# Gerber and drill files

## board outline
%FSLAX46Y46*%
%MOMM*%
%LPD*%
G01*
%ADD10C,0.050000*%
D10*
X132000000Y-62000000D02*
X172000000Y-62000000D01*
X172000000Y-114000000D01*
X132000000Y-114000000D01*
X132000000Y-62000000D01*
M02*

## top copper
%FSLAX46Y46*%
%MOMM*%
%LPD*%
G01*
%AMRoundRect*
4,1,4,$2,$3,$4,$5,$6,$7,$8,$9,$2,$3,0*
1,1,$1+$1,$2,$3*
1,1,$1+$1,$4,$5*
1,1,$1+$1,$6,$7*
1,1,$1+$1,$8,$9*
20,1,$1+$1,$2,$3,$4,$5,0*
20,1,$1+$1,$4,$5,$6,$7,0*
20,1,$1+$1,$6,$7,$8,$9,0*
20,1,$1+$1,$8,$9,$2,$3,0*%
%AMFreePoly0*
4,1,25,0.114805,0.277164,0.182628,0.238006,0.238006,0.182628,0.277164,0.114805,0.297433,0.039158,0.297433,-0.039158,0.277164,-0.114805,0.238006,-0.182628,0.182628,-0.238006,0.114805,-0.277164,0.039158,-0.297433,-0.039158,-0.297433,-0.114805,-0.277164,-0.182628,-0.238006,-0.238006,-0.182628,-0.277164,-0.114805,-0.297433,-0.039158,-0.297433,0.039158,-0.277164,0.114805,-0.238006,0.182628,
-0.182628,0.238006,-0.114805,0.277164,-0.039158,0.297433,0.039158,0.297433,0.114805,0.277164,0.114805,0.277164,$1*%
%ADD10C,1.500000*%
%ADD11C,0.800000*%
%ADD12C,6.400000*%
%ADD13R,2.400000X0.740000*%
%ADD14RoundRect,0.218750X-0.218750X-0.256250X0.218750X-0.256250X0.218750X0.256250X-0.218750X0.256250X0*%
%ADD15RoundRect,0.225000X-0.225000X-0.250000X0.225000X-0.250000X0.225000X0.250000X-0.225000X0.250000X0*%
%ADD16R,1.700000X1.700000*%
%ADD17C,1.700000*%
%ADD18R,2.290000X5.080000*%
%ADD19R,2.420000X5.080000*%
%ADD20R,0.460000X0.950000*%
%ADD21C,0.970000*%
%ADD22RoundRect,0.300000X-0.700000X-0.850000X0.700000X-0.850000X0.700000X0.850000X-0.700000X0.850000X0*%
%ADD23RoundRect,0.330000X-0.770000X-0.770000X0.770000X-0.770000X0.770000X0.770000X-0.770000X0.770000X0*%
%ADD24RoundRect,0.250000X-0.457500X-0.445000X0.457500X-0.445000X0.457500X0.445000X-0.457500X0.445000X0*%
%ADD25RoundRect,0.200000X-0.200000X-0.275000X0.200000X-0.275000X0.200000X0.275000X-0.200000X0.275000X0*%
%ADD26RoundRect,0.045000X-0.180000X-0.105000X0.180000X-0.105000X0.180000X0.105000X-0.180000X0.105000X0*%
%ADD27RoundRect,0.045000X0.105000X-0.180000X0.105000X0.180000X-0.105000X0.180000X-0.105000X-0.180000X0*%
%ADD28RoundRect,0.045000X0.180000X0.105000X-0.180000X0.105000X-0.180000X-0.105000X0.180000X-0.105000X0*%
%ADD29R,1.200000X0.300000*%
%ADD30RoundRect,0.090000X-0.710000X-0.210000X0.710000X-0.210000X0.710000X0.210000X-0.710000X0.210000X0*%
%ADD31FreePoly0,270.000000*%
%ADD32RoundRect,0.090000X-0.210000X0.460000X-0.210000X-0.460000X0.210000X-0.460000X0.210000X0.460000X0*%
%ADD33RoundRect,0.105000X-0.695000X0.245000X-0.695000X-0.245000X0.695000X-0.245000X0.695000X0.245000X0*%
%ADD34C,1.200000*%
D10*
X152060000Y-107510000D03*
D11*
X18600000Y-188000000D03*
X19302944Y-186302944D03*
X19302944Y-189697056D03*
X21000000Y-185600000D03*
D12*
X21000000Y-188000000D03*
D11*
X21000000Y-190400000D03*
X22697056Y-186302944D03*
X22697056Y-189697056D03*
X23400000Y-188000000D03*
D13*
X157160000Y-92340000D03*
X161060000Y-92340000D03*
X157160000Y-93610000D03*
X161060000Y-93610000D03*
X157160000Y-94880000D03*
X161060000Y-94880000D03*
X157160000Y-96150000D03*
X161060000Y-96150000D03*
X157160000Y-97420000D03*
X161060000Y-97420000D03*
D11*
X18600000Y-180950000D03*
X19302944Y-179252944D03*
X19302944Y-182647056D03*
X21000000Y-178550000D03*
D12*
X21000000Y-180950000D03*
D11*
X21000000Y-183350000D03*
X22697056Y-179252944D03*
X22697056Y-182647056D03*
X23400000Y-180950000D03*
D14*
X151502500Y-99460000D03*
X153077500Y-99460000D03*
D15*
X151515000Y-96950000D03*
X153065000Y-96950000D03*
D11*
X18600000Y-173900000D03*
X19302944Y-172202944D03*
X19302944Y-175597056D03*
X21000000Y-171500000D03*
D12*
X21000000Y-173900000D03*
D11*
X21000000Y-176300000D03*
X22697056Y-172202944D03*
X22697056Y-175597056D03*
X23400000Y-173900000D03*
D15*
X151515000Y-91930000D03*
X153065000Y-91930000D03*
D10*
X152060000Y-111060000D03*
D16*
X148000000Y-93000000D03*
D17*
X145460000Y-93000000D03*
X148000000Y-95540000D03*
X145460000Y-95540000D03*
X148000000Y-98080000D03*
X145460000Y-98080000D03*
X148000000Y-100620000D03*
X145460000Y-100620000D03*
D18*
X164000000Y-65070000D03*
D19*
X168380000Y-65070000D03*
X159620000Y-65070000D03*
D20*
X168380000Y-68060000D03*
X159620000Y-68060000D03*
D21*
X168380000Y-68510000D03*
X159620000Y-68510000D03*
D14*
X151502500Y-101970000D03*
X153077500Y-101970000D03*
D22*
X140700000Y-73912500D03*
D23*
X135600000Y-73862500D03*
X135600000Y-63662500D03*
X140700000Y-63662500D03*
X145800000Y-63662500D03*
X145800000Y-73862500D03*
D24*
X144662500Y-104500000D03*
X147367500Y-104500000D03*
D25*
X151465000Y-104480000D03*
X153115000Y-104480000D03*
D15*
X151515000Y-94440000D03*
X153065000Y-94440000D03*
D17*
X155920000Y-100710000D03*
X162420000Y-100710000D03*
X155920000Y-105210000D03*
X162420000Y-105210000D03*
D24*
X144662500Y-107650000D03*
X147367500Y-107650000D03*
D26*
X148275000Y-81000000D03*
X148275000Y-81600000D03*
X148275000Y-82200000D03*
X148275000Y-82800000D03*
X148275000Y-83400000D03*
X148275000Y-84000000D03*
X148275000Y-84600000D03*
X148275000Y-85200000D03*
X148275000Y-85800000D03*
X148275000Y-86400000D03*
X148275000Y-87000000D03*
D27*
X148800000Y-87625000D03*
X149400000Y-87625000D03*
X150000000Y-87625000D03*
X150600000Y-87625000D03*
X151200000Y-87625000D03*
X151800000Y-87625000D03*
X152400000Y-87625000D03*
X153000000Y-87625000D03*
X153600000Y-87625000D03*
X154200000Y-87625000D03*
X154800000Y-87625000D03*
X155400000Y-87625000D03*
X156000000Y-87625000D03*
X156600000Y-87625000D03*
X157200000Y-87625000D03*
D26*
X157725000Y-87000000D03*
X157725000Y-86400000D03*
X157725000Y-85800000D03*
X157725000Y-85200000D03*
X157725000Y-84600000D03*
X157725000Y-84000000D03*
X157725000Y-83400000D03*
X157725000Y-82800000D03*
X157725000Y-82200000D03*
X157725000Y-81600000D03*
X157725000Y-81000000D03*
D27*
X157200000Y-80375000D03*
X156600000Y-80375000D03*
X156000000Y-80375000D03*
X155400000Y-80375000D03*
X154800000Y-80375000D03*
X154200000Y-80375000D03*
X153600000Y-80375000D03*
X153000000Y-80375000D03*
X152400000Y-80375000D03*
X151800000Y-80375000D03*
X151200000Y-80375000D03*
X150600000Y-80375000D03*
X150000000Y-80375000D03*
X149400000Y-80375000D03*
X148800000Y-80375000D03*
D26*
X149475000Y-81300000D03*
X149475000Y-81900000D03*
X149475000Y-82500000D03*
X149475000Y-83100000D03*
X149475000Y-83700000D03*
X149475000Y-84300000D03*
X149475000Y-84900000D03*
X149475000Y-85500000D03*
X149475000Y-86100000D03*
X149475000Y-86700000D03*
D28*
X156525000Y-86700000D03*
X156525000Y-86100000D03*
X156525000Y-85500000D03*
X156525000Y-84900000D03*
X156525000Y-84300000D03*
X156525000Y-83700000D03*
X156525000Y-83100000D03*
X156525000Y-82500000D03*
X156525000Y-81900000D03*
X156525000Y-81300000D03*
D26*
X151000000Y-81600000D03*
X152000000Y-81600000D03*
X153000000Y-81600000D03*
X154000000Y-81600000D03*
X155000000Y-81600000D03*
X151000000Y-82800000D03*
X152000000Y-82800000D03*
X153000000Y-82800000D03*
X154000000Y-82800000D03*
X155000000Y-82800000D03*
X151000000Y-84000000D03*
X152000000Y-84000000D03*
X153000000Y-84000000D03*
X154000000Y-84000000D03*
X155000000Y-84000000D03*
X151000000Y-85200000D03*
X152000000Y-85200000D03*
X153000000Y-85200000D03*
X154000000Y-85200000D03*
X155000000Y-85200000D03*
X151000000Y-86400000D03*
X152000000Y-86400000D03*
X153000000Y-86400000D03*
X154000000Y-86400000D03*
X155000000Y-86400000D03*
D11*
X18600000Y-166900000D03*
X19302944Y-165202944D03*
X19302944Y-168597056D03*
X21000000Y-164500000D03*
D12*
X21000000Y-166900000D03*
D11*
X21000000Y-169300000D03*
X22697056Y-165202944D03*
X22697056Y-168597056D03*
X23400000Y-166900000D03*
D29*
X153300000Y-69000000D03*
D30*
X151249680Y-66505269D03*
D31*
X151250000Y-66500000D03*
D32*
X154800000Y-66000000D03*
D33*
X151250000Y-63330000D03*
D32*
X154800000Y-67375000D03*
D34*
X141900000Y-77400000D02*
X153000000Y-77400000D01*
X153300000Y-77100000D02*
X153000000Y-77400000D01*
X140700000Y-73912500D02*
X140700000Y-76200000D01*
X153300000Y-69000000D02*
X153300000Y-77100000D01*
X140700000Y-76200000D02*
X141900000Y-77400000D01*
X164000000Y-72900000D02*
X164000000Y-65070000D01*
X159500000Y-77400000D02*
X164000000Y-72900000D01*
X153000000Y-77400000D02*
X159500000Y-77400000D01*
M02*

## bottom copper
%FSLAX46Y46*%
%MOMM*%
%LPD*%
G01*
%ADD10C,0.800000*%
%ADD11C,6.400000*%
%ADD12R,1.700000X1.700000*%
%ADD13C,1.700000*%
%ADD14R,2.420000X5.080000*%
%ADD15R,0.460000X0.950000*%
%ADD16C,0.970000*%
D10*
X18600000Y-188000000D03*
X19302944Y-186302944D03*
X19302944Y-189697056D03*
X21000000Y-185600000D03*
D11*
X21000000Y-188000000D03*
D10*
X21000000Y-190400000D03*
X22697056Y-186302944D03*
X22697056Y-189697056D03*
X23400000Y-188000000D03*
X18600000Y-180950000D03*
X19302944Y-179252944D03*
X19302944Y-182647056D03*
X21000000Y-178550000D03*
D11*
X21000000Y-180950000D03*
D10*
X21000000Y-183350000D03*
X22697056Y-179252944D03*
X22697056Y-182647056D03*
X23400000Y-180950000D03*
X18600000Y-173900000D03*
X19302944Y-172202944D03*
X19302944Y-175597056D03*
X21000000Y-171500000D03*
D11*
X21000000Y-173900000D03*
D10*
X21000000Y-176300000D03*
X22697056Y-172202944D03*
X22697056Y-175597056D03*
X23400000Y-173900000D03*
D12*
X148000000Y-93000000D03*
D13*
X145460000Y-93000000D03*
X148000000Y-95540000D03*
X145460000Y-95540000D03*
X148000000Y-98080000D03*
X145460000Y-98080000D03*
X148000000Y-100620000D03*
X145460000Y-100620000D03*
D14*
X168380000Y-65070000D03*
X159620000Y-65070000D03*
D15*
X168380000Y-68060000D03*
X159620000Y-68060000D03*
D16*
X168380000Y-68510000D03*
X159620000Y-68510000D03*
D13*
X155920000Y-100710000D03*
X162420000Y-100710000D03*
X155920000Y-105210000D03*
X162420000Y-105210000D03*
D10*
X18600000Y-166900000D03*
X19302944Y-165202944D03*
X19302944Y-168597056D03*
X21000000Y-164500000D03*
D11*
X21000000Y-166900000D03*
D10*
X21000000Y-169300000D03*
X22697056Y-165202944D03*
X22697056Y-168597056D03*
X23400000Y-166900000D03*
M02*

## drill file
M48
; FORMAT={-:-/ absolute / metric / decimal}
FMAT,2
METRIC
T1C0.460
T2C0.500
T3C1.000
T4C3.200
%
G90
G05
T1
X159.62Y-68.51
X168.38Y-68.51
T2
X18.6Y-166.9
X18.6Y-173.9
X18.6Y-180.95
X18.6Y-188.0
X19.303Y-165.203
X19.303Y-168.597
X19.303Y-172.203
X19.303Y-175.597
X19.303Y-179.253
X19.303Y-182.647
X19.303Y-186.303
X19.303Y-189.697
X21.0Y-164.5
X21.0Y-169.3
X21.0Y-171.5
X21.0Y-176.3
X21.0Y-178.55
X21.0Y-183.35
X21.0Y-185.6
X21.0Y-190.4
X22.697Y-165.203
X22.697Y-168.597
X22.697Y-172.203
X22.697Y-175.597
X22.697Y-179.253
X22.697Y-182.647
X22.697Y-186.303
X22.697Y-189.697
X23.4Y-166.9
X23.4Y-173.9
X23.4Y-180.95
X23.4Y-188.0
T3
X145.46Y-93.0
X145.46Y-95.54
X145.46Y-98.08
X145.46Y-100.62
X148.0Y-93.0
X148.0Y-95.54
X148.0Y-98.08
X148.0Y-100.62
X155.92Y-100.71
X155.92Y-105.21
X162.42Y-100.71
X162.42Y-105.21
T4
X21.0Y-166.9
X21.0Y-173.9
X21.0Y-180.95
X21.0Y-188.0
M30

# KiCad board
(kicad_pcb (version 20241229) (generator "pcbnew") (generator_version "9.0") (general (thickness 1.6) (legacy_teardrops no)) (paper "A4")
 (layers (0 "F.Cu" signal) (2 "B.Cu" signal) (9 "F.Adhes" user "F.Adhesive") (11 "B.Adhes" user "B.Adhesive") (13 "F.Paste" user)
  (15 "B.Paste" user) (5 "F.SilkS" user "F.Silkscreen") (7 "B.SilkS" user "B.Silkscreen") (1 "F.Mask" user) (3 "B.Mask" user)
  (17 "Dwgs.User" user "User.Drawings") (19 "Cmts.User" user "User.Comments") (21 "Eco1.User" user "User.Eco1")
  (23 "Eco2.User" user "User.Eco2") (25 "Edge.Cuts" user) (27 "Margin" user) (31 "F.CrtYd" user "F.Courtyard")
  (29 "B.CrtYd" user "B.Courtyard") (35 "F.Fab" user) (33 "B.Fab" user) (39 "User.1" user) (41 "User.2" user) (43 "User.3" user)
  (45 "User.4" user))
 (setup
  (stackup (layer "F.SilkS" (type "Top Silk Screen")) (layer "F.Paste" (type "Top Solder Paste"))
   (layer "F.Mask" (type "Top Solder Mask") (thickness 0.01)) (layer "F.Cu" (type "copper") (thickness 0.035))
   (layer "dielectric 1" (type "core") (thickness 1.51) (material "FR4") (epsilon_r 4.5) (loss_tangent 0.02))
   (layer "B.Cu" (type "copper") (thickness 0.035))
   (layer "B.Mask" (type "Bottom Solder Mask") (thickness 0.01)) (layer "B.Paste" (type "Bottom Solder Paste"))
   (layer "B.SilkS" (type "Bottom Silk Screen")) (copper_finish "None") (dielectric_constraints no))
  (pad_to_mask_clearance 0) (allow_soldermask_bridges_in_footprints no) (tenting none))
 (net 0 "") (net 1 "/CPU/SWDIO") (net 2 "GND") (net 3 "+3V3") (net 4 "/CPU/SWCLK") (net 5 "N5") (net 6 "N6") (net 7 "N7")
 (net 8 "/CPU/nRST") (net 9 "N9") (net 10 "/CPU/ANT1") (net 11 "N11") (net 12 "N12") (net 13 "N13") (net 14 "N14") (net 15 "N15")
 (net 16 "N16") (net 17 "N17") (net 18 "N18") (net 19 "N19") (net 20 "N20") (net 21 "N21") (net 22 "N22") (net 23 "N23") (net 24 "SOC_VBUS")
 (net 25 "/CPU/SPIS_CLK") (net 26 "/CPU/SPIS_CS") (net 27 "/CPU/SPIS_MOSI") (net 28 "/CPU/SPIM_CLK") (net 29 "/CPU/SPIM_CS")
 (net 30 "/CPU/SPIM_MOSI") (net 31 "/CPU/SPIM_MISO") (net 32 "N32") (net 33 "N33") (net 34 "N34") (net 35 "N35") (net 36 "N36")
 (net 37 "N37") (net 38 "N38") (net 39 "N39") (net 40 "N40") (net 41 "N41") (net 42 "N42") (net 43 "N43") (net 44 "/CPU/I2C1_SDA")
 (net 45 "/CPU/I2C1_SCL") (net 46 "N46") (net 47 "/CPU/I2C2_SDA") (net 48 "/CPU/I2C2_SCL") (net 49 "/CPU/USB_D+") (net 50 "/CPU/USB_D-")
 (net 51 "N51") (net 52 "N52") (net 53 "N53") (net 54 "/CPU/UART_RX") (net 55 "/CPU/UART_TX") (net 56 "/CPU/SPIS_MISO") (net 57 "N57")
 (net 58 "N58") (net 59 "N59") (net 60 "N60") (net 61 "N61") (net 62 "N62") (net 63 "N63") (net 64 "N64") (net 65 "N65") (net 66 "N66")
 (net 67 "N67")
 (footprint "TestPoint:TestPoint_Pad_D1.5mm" (layer "F.Cu") (at 152.06 107.51)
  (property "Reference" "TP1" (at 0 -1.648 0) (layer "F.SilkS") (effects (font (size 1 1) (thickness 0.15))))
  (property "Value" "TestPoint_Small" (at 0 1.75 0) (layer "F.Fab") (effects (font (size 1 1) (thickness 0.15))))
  (pad "1" smd circle (at 0 0) (size 1.5 1.5) (layers "F.Cu" "F.Mask") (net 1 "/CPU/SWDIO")))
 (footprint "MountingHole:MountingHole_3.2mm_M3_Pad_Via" (layer "F.Cu") (at 21 188)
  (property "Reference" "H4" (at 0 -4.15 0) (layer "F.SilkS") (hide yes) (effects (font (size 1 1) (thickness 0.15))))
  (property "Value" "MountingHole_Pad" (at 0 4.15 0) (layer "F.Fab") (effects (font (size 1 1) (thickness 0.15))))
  (pad "1" thru_hole circle (at -2.4 0) (size 0.8 0.8) (drill 0.5) (layers "*.Cu" "*.Mask") (remove_unused_layers no) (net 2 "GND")
   (zone_connect 2))
  (pad "1" thru_hole circle (at -1.697056 -1.697056) (size 0.8 0.8) (drill 0.5) (layers "*.Cu" "*.Mask") (remove_unused_layers no)
   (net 2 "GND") (zone_connect 2))
  (pad "1" thru_hole circle (at -1.697056 1.697056) (size 0.8 0.8) (drill 0.5) (layers "*.Cu" "*.Mask") (remove_unused_layers no)
   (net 2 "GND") (zone_connect 2))
  (pad "1" thru_hole circle (at 0 -2.4) (size 0.8 0.8) (drill 0.5) (layers "*.Cu" "*.Mask") (remove_unused_layers no) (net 2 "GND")
   (zone_connect 2))
  (pad "1" thru_hole circle (at 0 0) (size 6.4 6.4) (drill 3.2) (layers "*.Cu" "*.Mask") (remove_unused_layers no) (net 2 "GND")
   (zone_connect 2))
  (pad "1" thru_hole circle (at 0 2.4) (size 0.8 0.8) (drill 0.5) (layers "*.Cu" "*.Mask") (remove_unused_layers no) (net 2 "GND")
   (zone_connect 2))
  (pad "1" thru_hole circle (at 1.697056 -1.697056) (size 0.8 0.8) (drill 0.5) (layers "*.Cu" "*.Mask") (remove_unused_layers no)
   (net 2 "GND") (zone_connect 2))
  (pad "1" thru_hole circle (at 1.697056 1.697056) (size 0.8 0.8) (drill 0.5) (layers "*.Cu" "*.Mask") (remove_unused_layers no)
   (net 2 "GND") (zone_connect 2))
  (pad "1" thru_hole circle (at 2.4 0) (size 0.8 0.8) (drill 0.5) (layers "*.Cu" "*.Mask") (remove_unused_layers no) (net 2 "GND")
   (zone_connect 2)))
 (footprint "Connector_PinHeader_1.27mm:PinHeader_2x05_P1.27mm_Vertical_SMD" (layer "F.Cu") (at 159.11 94.88)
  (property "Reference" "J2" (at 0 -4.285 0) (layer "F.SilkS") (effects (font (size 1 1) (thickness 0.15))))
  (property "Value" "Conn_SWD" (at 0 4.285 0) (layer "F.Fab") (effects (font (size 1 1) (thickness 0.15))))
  (pad "1" smd rect (at -1.95 -2.54) (size 2.4 0.74) (layers "F.Cu" "F.Mask" "F.Paste") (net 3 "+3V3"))
  (pad "2" smd rect (at 1.95 -2.54) (size 2.4 0.74) (layers "F.Cu" "F.Mask" "F.Paste") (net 1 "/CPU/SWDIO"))
  (pad "3" smd rect (at -1.95 -1.27) (size 2.4 0.74) (layers "F.Cu" "F.Mask" "F.Paste") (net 2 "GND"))
  (pad "4" smd rect (at 1.95 -1.27) (size 2.4 0.74) (layers "F.Cu" "F.Mask" "F.Paste") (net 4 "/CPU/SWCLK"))
  (pad "5" smd rect (at -1.95 0) (size 2.4 0.74) (layers "F.Cu" "F.Mask" "F.Paste") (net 2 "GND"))
  (pad "6" smd rect (at 1.95 0) (size 2.4 0.74) (layers "F.Cu" "F.Mask" "F.Paste") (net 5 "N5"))
  (pad "7" smd rect (at -1.95 1.27) (size 2.4 0.74) (layers "F.Cu" "F.Mask" "F.Paste") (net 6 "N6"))
  (pad "8" smd rect (at 1.95 1.27) (size 2.4 0.74) (layers "F.Cu" "F.Mask" "F.Paste") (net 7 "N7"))
  (pad "9" smd rect (at -1.95 2.54) (size 2.4 0.74) (layers "F.Cu" "F.Mask" "F.Paste") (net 2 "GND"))
  (pad "10" smd rect (at 1.95 2.54) (size 2.4 0.74) (layers "F.Cu" "F.Mask" "F.Paste") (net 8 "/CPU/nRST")))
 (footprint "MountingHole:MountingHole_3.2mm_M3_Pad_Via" (layer "F.Cu") (at 21 180.95)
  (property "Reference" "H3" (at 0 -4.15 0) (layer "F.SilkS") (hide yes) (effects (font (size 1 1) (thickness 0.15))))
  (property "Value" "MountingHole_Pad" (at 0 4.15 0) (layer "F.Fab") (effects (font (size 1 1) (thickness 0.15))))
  (pad "1" thru_hole circle (at -2.4 0) (size 0.8 0.8) (drill 0.5) (layers "*.Cu" "*.Mask") (remove_unused_layers no) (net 2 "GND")
   (zone_connect 2))
  (pad "1" thru_hole circle (at -1.697056 -1.697056) (size 0.8 0.8) (drill 0.5) (layers "*.Cu" "*.Mask") (remove_unused_layers no)
   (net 2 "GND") (zone_connect 2))
  (pad "1" thru_hole circle (at -1.697056 1.697056) (size 0.8 0.8) (drill 0.5) (layers "*.Cu" "*.Mask") (remove_unused_layers no)
   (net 2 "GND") (zone_connect 2))
  (pad "1" thru_hole circle (at 0 -2.4) (size 0.8 0.8) (drill 0.5) (layers "*.Cu" "*.Mask") (remove_unused_layers no) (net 2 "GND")
   (zone_connect 2))
  (pad "1" thru_hole circle (at 0 0) (size 6.4 6.4) (drill 3.2) (layers "*.Cu" "*.Mask") (remove_unused_layers no) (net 2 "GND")
   (zone_connect 2))
  (pad "1" thru_hole circle (at 0 2.4) (size 0.8 0.8) (drill 0.5) (layers "*.Cu" "*.Mask") (remove_unused_layers no) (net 2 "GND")
   (zone_connect 2))
  (pad "1" thru_hole circle (at 1.697056 -1.697056) (size 0.8 0.8) (drill 0.5) (layers "*.Cu" "*.Mask") (remove_unused_layers no)
   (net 2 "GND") (zone_connect 2))
  (pad "1" thru_hole circle (at 1.697056 1.697056) (size 0.8 0.8) (drill 0.5) (layers "*.Cu" "*.Mask") (remove_unused_layers no)
   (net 2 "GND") (zone_connect 2))
  (pad "1" thru_hole circle (at 2.4 0) (size 0.8 0.8) (drill 0.5) (layers "*.Cu" "*.Mask") (remove_unused_layers no) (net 2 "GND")
   (zone_connect 2)))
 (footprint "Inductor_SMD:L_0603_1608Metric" (layer "F.Cu") (at 152.29 99.46)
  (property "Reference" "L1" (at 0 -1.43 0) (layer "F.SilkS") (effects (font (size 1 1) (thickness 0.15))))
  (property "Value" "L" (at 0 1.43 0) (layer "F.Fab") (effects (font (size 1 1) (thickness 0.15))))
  (pad "1" smd roundrect (at -0.7875 0) (size 0.875 0.95) (layers "F.Cu" "F.Mask" "F.Paste") (roundrect_rratio 0.25) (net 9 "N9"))
  (pad "2" smd roundrect (at 0.7875 0) (size 0.875 0.95) (layers "F.Cu" "F.Mask" "F.Paste") (roundrect_rratio 0.25) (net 2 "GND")))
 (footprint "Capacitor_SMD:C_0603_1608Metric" (layer "F.Cu") (at 152.29 96.95)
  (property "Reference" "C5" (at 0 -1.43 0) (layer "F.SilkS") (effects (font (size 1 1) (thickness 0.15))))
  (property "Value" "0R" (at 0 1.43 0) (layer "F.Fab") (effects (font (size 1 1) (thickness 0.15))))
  (pad "1" smd roundrect (at -0.775 0) (size 0.9 0.95) (layers "F.Cu" "F.Mask" "F.Paste") (roundrect_rratio 0.25) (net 9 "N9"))
  (pad "2" smd roundrect (at 0.775 0) (size 0.9 0.95) (layers "F.Cu" "F.Mask" "F.Paste") (roundrect_rratio 0.25) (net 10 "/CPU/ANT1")))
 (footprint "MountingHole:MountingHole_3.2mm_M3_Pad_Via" (layer "F.Cu") (at 21 173.9)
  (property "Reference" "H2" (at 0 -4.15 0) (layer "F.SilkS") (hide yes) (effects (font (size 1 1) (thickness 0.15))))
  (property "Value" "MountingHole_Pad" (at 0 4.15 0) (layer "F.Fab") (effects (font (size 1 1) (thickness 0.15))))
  (pad "1" thru_hole circle (at -2.4 0) (size 0.8 0.8) (drill 0.5) (layers "*.Cu" "*.Mask") (remove_unused_layers no) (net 2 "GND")
   (zone_connect 2))
  (pad "1" thru_hole circle (at -1.697056 -1.697056) (size 0.8 0.8) (drill 0.5) (layers "*.Cu" "*.Mask") (remove_unused_layers no)
   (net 2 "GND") (zone_connect 2))
  (pad "1" thru_hole circle (at -1.697056 1.697056) (size 0.8 0.8) (drill 0.5) (layers "*.Cu" "*.Mask") (remove_unused_layers no)
   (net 2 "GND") (zone_connect 2))
  (pad "1" thru_hole circle (at 0 -2.4) (size 0.8 0.8) (drill 0.5) (layers "*.Cu" "*.Mask") (remove_unused_layers no) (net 2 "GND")
   (zone_connect 2))
  (pad "1" thru_hole circle (at 0 0) (size 6.4 6.4) (drill 3.2) (layers "*.Cu" "*.Mask") (remove_unused_layers no) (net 2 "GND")
   (zone_connect 2))
  (pad "1" thru_hole circle (at 0 2.4) (size 0.8 0.8) (drill 0.5) (layers "*.Cu" "*.Mask") (remove_unused_layers no) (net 2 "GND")
   (zone_connect 2))
  (pad "1" thru_hole circle (at 1.697056 -1.697056) (size 0.8 0.8) (drill 0.5) (layers "*.Cu" "*.Mask") (remove_unused_layers no)
   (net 2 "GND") (zone_connect 2))
  (pad "1" thru_hole circle (at 1.697056 1.697056) (size 0.8 0.8) (drill 0.5) (layers "*.Cu" "*.Mask") (remove_unused_layers no)
   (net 2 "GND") (zone_connect 2))
  (pad "1" thru_hole circle (at 2.4 0) (size 0.8 0.8) (drill 0.5) (layers "*.Cu" "*.Mask") (remove_unused_layers no) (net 2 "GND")
   (zone_connect 2)))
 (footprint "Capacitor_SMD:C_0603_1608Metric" (layer "F.Cu") (at 152.29 91.93)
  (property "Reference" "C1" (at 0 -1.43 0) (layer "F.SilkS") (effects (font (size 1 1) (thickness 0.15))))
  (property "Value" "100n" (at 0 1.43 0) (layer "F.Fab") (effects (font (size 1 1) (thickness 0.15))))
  (pad "1" smd roundrect (at -0.775 0) (size 0.9 0.95) (layers "F.Cu" "F.Mask" "F.Paste") (roundrect_rratio 0.25) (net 3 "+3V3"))
  (pad "2" smd roundrect (at 0.775 0) (size 0.9 0.95) (layers "F.Cu" "F.Mask" "F.Paste") (roundrect_rratio 0.25) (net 2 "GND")))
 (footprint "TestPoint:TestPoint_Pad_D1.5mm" (layer "F.Cu") (at 152.06 111.06)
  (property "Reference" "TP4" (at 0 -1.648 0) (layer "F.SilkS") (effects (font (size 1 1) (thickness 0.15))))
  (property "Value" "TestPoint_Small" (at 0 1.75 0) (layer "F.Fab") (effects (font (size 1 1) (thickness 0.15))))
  (pad "1" smd circle (at 0 0) (size 1.5 1.5) (layers "F.Cu" "F.Mask") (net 4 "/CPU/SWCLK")))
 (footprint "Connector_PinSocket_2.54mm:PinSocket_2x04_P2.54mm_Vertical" (layer "F.Cu") (at 148 93)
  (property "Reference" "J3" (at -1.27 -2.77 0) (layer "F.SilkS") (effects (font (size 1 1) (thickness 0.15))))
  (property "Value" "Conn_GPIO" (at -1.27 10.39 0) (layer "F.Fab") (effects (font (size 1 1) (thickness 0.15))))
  (pad "1" thru_hole rect (at 0 0) (size 1.7 1.7) (drill 1) (layers "*.Cu" "*.Mask") (remove_unused_layers no) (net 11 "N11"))
  (pad "2" thru_hole circle (at -2.54 0) (size 1.7 1.7) (drill 1) (layers "*.Cu" "*.Mask") (remove_unused_layers no) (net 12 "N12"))
  (pad "3" thru_hole circle (at 0 2.54) (size 1.7 1.7) (drill 1) (layers "*.Cu" "*.Mask") (remove_unused_layers no) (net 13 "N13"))
  (pad "4" thru_hole circle (at -2.54 2.54) (size 1.7 1.7) (drill 1) (layers "*.Cu" "*.Mask") (remove_unused_layers no) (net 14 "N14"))
  (pad "5" thru_hole circle (at 0 5.08) (size 1.7 1.7) (drill 1) (layers "*.Cu" "*.Mask") (remove_unused_layers no) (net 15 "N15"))
  (pad "6" thru_hole circle (at -2.54 5.08) (size 1.7 1.7) (drill 1) (layers "*.Cu" "*.Mask") (remove_unused_layers no) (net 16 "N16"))
  (pad "7" thru_hole circle (at 0 7.62) (size 1.7 1.7) (drill 1) (layers "*.Cu" "*.Mask") (remove_unused_layers no) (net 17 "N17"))
  (pad "8" thru_hole circle (at -2.54 7.62) (size 1.7 1.7) (drill 1) (layers "*.Cu" "*.Mask") (remove_unused_layers no) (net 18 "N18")))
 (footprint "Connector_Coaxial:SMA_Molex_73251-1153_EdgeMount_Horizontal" (layer "F.Cu") (at 164 66.79 -90)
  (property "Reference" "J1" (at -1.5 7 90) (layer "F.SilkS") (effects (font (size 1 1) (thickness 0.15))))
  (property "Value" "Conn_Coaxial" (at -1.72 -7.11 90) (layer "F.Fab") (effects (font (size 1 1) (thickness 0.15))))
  (pad "1" smd rect (at -1.72 0 270) (size 5.08 2.29) (layers "F.Cu" "F.Mask" "F.Paste") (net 10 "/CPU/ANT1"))
  (pad "2" smd rect (at -1.72 -4.38 270) (size 5.08 2.42) (layers "F.Cu" "F.Mask" "F.Paste") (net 2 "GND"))
  (pad "2" smd rect (at -1.72 -4.38 270) (size 5.08 2.42) (layers "B.Cu" "B.Mask" "B.Paste") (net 2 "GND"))
  (pad "2" smd rect (at -1.72 4.38 270) (size 5.08 2.42) (layers "F.Cu" "F.Mask" "F.Paste") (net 2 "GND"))
  (pad "2" smd rect (at -1.72 4.38 270) (size 5.08 2.42) (layers "B.Cu" "B.Mask" "B.Paste") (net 2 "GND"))
  (pad "2" smd rect (at 1.27 -4.38 270) (size 0.95 0.46) (layers "F.Cu") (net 2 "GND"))
  (pad "2" smd rect (at 1.27 -4.38 270) (size 0.95 0.46) (layers "B.Cu") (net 2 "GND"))
  (pad "2" smd rect (at 1.27 4.38 270) (size 0.95 0.46) (layers "F.Cu") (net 2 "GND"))
  (pad "2" smd rect (at 1.27 4.38 270) (size 0.95 0.46) (layers "B.Cu") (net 2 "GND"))
  (pad "2" thru_hole circle (at 1.72 -4.38 270) (size 0.97 0.97) (drill 0.46) (layers "*.Cu") (remove_unused_layers no) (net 2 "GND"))
  (pad "2" thru_hole circle (at 1.72 4.38 270) (size 0.97 0.97) (drill 0.46) (layers "*.Cu") (remove_unused_layers no) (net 2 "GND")))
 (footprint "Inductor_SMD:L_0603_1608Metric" (layer "F.Cu") (at 152.29 101.97)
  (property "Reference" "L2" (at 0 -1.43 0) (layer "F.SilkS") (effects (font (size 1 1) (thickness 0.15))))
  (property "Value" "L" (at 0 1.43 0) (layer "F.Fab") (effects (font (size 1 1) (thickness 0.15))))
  (pad "1" smd roundrect (at -0.7875 0) (size 0.875 0.95) (layers "F.Cu" "F.Mask" "F.Paste") (roundrect_rratio 0.25) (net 10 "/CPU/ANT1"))
  (pad "2" smd roundrect (at 0.7875 0) (size 0.875 0.95) (layers "F.Cu" "F.Mask" "F.Paste") (roundrect_rratio 0.25) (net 2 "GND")))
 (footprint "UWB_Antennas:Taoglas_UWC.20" (layer "F.Cu") (at 140.7 68.7625)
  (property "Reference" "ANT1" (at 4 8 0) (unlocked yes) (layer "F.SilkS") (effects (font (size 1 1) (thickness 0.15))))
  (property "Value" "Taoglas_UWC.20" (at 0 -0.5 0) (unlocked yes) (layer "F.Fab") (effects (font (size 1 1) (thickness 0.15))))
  (pad "1" smd roundrect (at 0 5.15) (size 2 2.3) (layers "F.Cu" "F.Mask" "F.Paste") (roundrect_rratio 0.15) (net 10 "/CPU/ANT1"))
  (pad "2" smd roundrect (at -5.1 5.1) (size 2.2 2.2) (layers "F.Cu" "F.Mask" "F.Paste") (roundrect_rratio 0.15) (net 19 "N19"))
  (pad "3" smd roundrect (at -5.1 -5.1) (size 2.2 2.2) (layers "F.Cu" "F.Mask" "F.Paste") (roundrect_rratio 0.15) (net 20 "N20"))
  (pad "4" smd roundrect (at 0 -5.1) (size 2.2 2.2) (layers "F.Cu" "F.Mask" "F.Paste") (roundrect_rratio 0.15) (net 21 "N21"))
  (pad "5" smd roundrect (at 5.1 -5.1) (size 2.2 2.2) (layers "F.Cu" "F.Mask" "F.Paste") (roundrect_rratio 0.15) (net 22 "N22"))
  (pad "6" smd roundrect (at 5.1 5.1) (size 2.2 2.2) (layers "F.Cu" "F.Mask" "F.Paste") (roundrect_rratio 0.15) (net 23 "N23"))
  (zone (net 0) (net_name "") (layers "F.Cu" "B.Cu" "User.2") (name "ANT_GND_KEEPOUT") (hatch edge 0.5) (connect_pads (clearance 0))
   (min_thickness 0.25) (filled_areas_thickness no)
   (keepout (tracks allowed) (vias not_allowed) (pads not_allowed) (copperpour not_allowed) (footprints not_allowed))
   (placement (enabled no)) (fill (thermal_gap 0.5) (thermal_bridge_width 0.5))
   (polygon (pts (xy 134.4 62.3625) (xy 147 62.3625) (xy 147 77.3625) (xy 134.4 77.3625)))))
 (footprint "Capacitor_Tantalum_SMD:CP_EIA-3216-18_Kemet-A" (layer "F.Cu") (at 146.015 104.5)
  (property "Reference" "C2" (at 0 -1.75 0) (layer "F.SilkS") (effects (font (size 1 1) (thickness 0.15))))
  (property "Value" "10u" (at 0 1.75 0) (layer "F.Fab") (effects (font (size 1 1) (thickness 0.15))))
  (pad "1" smd roundrect (at -1.3525 0) (size 1.415 1.39) (layers "F.Cu" "F.Mask" "F.Paste") (roundrect_rratio 0.179856) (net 3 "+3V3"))
  (pad "2" smd roundrect (at 1.3525 0) (size 1.415 1.39) (layers "F.Cu" "F.Mask" "F.Paste") (roundrect_rratio 0.179856) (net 2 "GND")))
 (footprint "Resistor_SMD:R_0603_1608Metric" (layer "F.Cu") (at 152.29 104.48)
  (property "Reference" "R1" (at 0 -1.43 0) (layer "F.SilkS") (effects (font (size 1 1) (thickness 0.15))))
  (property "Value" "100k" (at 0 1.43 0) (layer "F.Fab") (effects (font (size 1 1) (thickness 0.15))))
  (pad "1" smd roundrect (at -0.825 0) (size 0.8 0.95) (layers "F.Cu" "F.Mask" "F.Paste") (roundrect_rratio 0.25) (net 3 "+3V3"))
  (pad "2" smd roundrect (at 0.825 0) (size 0.8 0.95) (layers "F.Cu" "F.Mask" "F.Paste") (roundrect_rratio 0.25) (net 8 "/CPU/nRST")))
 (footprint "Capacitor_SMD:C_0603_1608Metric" (layer "F.Cu") (at 152.29 94.44)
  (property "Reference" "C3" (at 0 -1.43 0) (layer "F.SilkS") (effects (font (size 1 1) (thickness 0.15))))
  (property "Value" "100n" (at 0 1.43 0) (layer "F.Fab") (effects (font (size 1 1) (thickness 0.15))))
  (pad "1" smd roundrect (at -0.775 0) (size 0.9 0.95) (layers "F.Cu" "F.Mask" "F.Paste") (roundrect_rratio 0.25) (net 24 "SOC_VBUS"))
  (pad "2" smd roundrect (at 0.775 0) (size 0.9 0.95) (layers "F.Cu" "F.Mask" "F.Paste") (roundrect_rratio 0.25) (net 2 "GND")))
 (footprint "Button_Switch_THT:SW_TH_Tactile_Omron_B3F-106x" (layer "F.Cu") (at 155.92 100.71)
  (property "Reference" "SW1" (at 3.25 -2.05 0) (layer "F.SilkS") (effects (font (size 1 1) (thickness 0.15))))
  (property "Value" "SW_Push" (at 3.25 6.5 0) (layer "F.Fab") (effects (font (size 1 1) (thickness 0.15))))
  (pad "1" thru_hole circle (at 0 0) (size 1.7 1.7) (drill 1) (layers "*.Cu" "*.Mask") (remove_unused_layers no) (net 2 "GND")
   (thermal_bridge_angle 90))
  (pad "1" thru_hole circle (at 6.5 0) (size 1.7 1.7) (drill 1) (layers "*.Cu" "*.Mask") (remove_unused_layers no) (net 2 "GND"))
  (pad "2" thru_hole circle (at 0 4.5) (size 1.7 1.7) (drill 1) (layers "*.Cu" "*.Mask") (remove_unused_layers no) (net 8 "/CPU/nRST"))
  (pad "2" thru_hole circle (at 6.5 4.5) (size 1.7 1.7) (drill 1) (layers "*.Cu" "*.Mask") (remove_unused_layers no) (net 8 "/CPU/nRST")))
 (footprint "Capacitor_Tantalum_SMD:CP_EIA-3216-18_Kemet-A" (layer "F.Cu") (at 146.015 107.65)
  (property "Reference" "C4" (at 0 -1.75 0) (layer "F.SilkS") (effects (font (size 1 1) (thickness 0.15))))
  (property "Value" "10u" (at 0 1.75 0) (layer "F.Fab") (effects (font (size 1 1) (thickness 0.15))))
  (pad "1" smd roundrect (at -1.3525 0) (size 1.415 1.39) (layers "F.Cu" "F.Mask" "F.Paste") (roundrect_rratio 0.179856) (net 24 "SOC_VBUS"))
  (pad "2" smd roundrect (at 1.3525 0) (size 1.415 1.39) (layers "F.Cu" "F.Mask" "F.Paste") (roundrect_rratio 0.179856) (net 2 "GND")))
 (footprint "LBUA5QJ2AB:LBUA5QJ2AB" (layer "F.Cu") (at 153 84)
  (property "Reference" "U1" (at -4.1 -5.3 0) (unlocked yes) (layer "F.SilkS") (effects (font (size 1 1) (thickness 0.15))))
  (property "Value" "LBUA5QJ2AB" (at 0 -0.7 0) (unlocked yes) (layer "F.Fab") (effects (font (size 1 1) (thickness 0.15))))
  (pad "1" smd roundrect (at -4.725 -3) (size 0.45 0.3) (layers "F.Cu" "F.Mask" "F.Paste") (roundrect_rratio 0.15) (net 2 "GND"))
  (pad "2" smd roundrect (at -4.725 -2.4) (size 0.45 0.3) (layers "F.Cu" "F.Mask" "F.Paste") (roundrect_rratio 0.15)
   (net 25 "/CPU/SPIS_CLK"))
  (pad "3" smd roundrect (at -4.725 -1.8) (size 0.45 0.3) (layers "F.Cu" "F.Mask" "F.Paste") (roundrect_rratio 0.15) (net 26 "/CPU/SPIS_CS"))
  (pad "4" smd roundrect (at -4.725 -1.2) (size 0.45 0.3) (layers "F.Cu" "F.Mask" "F.Paste") (roundrect_rratio 0.15)
   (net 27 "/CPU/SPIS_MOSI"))
  (pad "5" smd roundrect (at -4.725 -0.6) (size 0.45 0.3) (layers "F.Cu" "F.Mask" "F.Paste") (roundrect_rratio 0.15)
   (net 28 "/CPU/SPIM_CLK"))
  (pad "6" smd roundrect (at -4.725 0) (size 0.45 0.3) (layers "F.Cu" "F.Mask" "F.Paste") (roundrect_rratio 0.15) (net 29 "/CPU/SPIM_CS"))
  (pad "7" smd roundrect (at -4.725 0.6) (size 0.45 0.3) (layers "F.Cu" "F.Mask" "F.Paste") (roundrect_rratio 0.15)
   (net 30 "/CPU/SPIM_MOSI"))
  (pad "8" smd roundrect (at -4.725 1.2) (size 0.45 0.3) (layers "F.Cu" "F.Mask" "F.Paste") (roundrect_rratio 0.15)
   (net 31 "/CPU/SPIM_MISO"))
  (pad "9" smd roundrect (at -4.725 1.8) (size 0.45 0.3) (layers "F.Cu" "F.Mask" "F.Paste") (roundrect_rratio 0.15) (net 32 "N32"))
  (pad "10" smd roundrect (at -4.725 2.4) (size 0.45 0.3) (layers "F.Cu" "F.Mask" "F.Paste") (roundrect_rratio 0.15) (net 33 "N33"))
  (pad "11" smd roundrect (at -4.725 3) (size 0.45 0.3) (layers "F.Cu" "F.Mask" "F.Paste") (roundrect_rratio 0.15) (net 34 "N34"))
  (pad "12" smd roundrect (at -4.2 3.625 90) (size 0.45 0.3) (layers "F.Cu" "F.Mask" "F.Paste") (roundrect_rratio 0.15) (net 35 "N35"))
  (pad "13" smd roundrect (at -3.6 3.625 90) (size 0.45 0.3) (layers "F.Cu" "F.Mask" "F.Paste") (roundrect_rratio 0.15) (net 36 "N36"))
  (pad "14" smd roundrect (at -3 3.625 90) (size 0.45 0.3) (layers "F.Cu" "F.Mask" "F.Paste") (roundrect_rratio 0.15) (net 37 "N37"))
  (pad "15" smd roundrect (at -2.4 3.625 90) (size 0.45 0.3) (layers "F.Cu" "F.Mask" "F.Paste") (roundrect_rratio 0.15) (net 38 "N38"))
  (pad "16" smd roundrect (at -1.8 3.625 90) (size 0.45 0.3) (layers "F.Cu" "F.Mask" "F.Paste") (roundrect_rratio 0.15) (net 2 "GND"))
  (pad "17" smd roundrect (at -1.2 3.625 90) (size 0.45 0.3) (layers "F.Cu" "F.Mask" "F.Paste") (roundrect_rratio 0.15) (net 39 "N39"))
  (pad "18" smd roundrect (at -0.6 3.625 90) (size 0.45 0.3) (layers "F.Cu" "F.Mask" "F.Paste") (roundrect_rratio 0.15) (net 2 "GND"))
  (pad "19" smd roundrect (at 0 3.625 90) (size 0.45 0.3) (layers "F.Cu" "F.Mask" "F.Paste") (roundrect_rratio 0.15) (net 2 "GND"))
  (pad "20" smd roundrect (at 0.6 3.625 90) (size 0.45 0.3) (layers "F.Cu" "F.Mask" "F.Paste") (roundrect_rratio 0.15) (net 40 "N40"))
  (pad "21" smd roundrect (at 1.2 3.625 90) (size 0.45 0.3) (layers "F.Cu" "F.Mask" "F.Paste") (roundrect_rratio 0.15) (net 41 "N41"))
  (pad "22" smd roundrect (at 1.8 3.625 90) (size 0.45 0.3) (layers "F.Cu" "F.Mask" "F.Paste") (roundrect_rratio 0.15) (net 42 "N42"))
  (pad "23" smd roundrect (at 2.4 3.625 90) (size 0.45 0.3) (layers "F.Cu" "F.Mask" "F.Paste") (roundrect_rratio 0.15) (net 2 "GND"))
  (pad "24" smd roundrect (at 3 3.625 90) (size 0.45 0.3) (layers "F.Cu" "F.Mask" "F.Paste") (roundrect_rratio 0.15) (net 4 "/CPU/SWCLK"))
  (pad "25" smd roundrect (at 3.6 3.625 90) (size 0.45 0.3) (layers "F.Cu" "F.Mask" "F.Paste") (roundrect_rratio 0.15) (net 1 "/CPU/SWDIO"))
  (pad "26" smd roundrect (at 4.2 3.625 90) (size 0.45 0.3) (layers "F.Cu" "F.Mask" "F.Paste") (roundrect_rratio 0.15) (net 2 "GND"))
  (pad "27" smd roundrect (at 4.725 3) (size 0.45 0.3) (layers "F.Cu" "F.Mask" "F.Paste") (roundrect_rratio 0.15) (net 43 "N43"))
  (pad "28" smd roundrect (at 4.725 2.4) (size 0.45 0.3) (layers "F.Cu" "F.Mask" "F.Paste") (roundrect_rratio 0.15) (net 2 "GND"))
  (pad "29" smd roundrect (at 4.725 1.8) (size 0.45 0.3) (layers "F.Cu" "F.Mask" "F.Paste") (roundrect_rratio 0.15) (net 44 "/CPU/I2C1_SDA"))
  (pad "30" smd roundrect (at 4.725 1.2) (size 0.45 0.3) (layers "F.Cu" "F.Mask" "F.Paste") (roundrect_rratio 0.15) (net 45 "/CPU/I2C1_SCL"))
  (pad "31" smd roundrect (at 4.725 0.6) (size 0.45 0.3) (layers "F.Cu" "F.Mask" "F.Paste") (roundrect_rratio 0.15) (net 2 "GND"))
  (pad "32" smd roundrect (at 4.725 0) (size 0.45 0.3) (layers "F.Cu" "F.Mask" "F.Paste") (roundrect_rratio 0.15) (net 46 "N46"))
  (pad "33" smd roundrect (at 4.725 -0.6) (size 0.45 0.3) (layers "F.Cu" "F.Mask" "F.Paste") (roundrect_rratio 0.15)
   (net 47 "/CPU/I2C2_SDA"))
  (pad "34" smd roundrect (at 4.725 -1.2) (size 0.45 0.3) (layers "F.Cu" "F.Mask" "F.Paste") (roundrect_rratio 0.15)
   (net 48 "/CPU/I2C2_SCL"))
  (pad "35" smd roundrect (at 4.725 -1.8) (size 0.45 0.3) (layers "F.Cu" "F.Mask" "F.Paste") (roundrect_rratio 0.15) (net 8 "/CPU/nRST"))
  (pad "36" smd roundrect (at 4.725 -2.4) (size 0.45 0.3) (layers "F.Cu" "F.Mask" "F.Paste") (roundrect_rratio 0.15) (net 2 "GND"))
  (pad "37" smd roundrect (at 4.725 -3) (size 0.45 0.3) (layers "F.Cu" "F.Mask" "F.Paste") (roundrect_rratio 0.15) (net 9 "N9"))
  (pad "38" smd roundrect (at 4.2 -3.625 90) (size 0.45 0.3) (layers "F.Cu" "F.Mask" "F.Paste") (roundrect_rratio 0.15) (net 2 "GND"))
  (pad "39" smd roundrect (at 3.6 -3.625 90) (size 0.45 0.3) (layers "F.Cu" "F.Mask" "F.Paste") (roundrect_rratio 0.15)
   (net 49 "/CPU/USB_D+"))
  (pad "40" smd roundrect (at 3 -3.625 90) (size 0.45 0.3) (layers "F.Cu" "F.Mask" "F.Paste") (roundrect_rratio 0.15) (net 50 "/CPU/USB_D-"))
  (pad "41" smd roundrect (at 2.4 -3.625 90) (size 0.45 0.3) (layers "F.Cu" "F.Mask" "F.Paste") (roundrect_rratio 0.15) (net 2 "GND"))
  (pad "42" smd roundrect (at 1.8 -3.625 90) (size 0.45 0.3) (layers "F.Cu" "F.Mask" "F.Paste") (roundrect_rratio 0.15) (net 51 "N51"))
  (pad "43" smd roundrect (at 1.2 -3.625 90) (size 0.45 0.3) (layers "F.Cu" "F.Mask" "F.Paste") (roundrect_rratio 0.15) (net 3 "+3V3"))
  (pad "44" smd roundrect (at 0.6 -3.625 90) (size 0.45 0.3) (layers "F.Cu" "F.Mask" "F.Paste") (roundrect_rratio 0.15) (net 3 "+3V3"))
  (pad "45" smd roundrect (at 0 -3.625 90) (size 0.45 0.3) (layers "F.Cu" "F.Mask" "F.Paste") (roundrect_rratio 0.15) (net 24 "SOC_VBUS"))
  (pad "46" smd roundrect (at -0.6 -3.625 90) (size 0.45 0.3) (layers "F.Cu" "F.Mask" "F.Paste") (roundrect_rratio 0.15) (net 3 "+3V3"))
  (pad "47" smd roundrect (at -1.2 -3.625 90) (size 0.45 0.3) (layers "F.Cu" "F.Mask" "F.Paste") (roundrect_rratio 0.15) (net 2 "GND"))
  (pad "48" smd roundrect (at -1.8 -3.625 90) (size 0.45 0.3) (layers "F.Cu" "F.Mask" "F.Paste") (roundrect_rratio 0.15) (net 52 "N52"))
  (pad "49" smd roundrect (at -2.4 -3.625 90) (size 0.45 0.3) (layers "F.Cu" "F.Mask" "F.Paste") (roundrect_rratio 0.15) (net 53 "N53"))
  (pad "50" smd roundrect (at -3 -3.625 90) (size 0.45 0.3) (layers "F.Cu" "F.Mask" "F.Paste") (roundrect_rratio 0.15)
   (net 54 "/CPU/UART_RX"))
  (pad "51" smd roundrect (at -3.6 -3.625 90) (size 0.45 0.3) (layers "F.Cu" "F.Mask" "F.Paste") (roundrect_rratio 0.15)
   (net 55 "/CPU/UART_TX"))
  (pad "52" smd roundrect (at -4.2 -3.625 90) (size 0.45 0.3) (layers "F.Cu" "F.Mask" "F.Paste") (roundrect_rratio 0.15)
   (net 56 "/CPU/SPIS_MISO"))
  (pad "53" smd roundrect (at -3.525 -2.7) (size 0.45 0.3) (layers "F.Cu" "F.Mask" "F.Paste") (roundrect_rratio 0.15) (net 2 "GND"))
  (pad "54" smd roundrect (at -3.525 -2.1) (size 0.45 0.3) (layers "F.Cu" "F.Mask" "F.Paste") (roundrect_rratio 0.15) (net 11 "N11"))
  (pad "55" smd roundrect (at -3.525 -1.5) (size 0.45 0.3) (layers "F.Cu" "F.Mask" "F.Paste") (roundrect_rratio 0.15) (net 12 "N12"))
  (pad "56" smd roundrect (at -3.525 -0.9) (size 0.45 0.3) (layers "F.Cu" "F.Mask" "F.Paste") (roundrect_rratio 0.15) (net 13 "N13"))
  (pad "57" smd roundrect (at -3.525 -0.3) (size 0.45 0.3) (layers "F.Cu" "F.Mask" "F.Paste") (roundrect_rratio 0.15) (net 14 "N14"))
  (pad "58" smd roundrect (at -3.525 0.3) (size 0.45 0.3) (layers "F.Cu" "F.Mask" "F.Paste") (roundrect_rratio 0.15) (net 15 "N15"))
  (pad "59" smd roundrect (at -3.525 0.9) (size 0.45 0.3) (layers "F.Cu" "F.Mask" "F.Paste") (roundrect_rratio 0.15) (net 16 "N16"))
  (pad "60" smd roundrect (at -3.525 1.5) (size 0.45 0.3) (layers "F.Cu" "F.Mask" "F.Paste") (roundrect_rratio 0.15) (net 17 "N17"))
  (pad "61" smd roundrect (at -3.525 2.1) (size 0.45 0.3) (layers "F.Cu" "F.Mask" "F.Paste") (roundrect_rratio 0.15) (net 18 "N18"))
  (pad "62" smd roundrect (at -3.525 2.7) (size 0.45 0.3) (layers "F.Cu" "F.Mask" "F.Paste") (roundrect_rratio 0.15) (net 2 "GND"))
  (pad "63" smd roundrect (at 3.525 2.7 180) (size 0.45 0.3) (layers "F.Cu" "F.Mask" "F.Paste") (roundrect_rratio 0.15) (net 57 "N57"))
  (pad "64" smd roundrect (at 3.525 2.1 180) (size 0.45 0.3) (layers "F.Cu" "F.Mask" "F.Paste") (roundrect_rratio 0.15) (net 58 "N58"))
  (pad "65" smd roundrect (at 3.525 1.5 180) (size 0.45 0.3) (layers "F.Cu" "F.Mask" "F.Paste") (roundrect_rratio 0.15) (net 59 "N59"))
  (pad "66" smd roundrect (at 3.525 0.9 180) (size 0.45 0.3) (layers "F.Cu" "F.Mask" "F.Paste") (roundrect_rratio 0.15) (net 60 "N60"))
  (pad "67" smd roundrect (at 3.525 0.3 180) (size 0.45 0.3) (layers "F.Cu" "F.Mask" "F.Paste") (roundrect_rratio 0.15) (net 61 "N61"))
  (pad "68" smd roundrect (at 3.525 -0.3 180) (size 0.45 0.3) (layers "F.Cu" "F.Mask" "F.Paste") (roundrect_rratio 0.15) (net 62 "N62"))
  (pad "69" smd roundrect (at 3.525 -0.9 180) (size 0.45 0.3) (layers "F.Cu" "F.Mask" "F.Paste") (roundrect_rratio 0.15) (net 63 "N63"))
  (pad "70" smd roundrect (at 3.525 -1.5 180) (size 0.45 0.3) (layers "F.Cu" "F.Mask" "F.Paste") (roundrect_rratio 0.15) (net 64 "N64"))
  (pad "71" smd roundrect (at 3.525 -2.1 180) (size 0.45 0.3) (layers "F.Cu" "F.Mask" "F.Paste") (roundrect_rratio 0.15) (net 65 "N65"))
  (pad "72" smd roundrect (at 3.525 -2.7 180) (size 0.45 0.3) (layers "F.Cu" "F.Mask" "F.Paste") (roundrect_rratio 0.15) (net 2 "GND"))
  (pad "73" smd roundrect (at -2 -2.4) (size 0.45 0.3) (layers "F.Cu" "F.Mask" "F.Paste") (roundrect_rratio 0.15) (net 2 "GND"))
  (pad "74" smd roundrect (at -1 -2.4) (size 0.45 0.3) (layers "F.Cu" "F.Mask" "F.Paste") (roundrect_rratio 0.15) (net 2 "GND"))
  (pad "75" smd roundrect (at 0 -2.4) (size 0.45 0.3) (layers "F.Cu" "F.Mask" "F.Paste") (roundrect_rratio 0.15) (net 2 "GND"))
  (pad "76" smd roundrect (at 1 -2.4) (size 0.45 0.3) (layers "F.Cu" "F.Mask" "F.Paste") (roundrect_rratio 0.15) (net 2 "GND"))
  (pad "77" smd roundrect (at 2 -2.4) (size 0.45 0.3) (layers "F.Cu" "F.Mask" "F.Paste") (roundrect_rratio 0.15) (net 2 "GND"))
  (pad "78" smd roundrect (at -2 -1.2) (size 0.45 0.3) (layers "F.Cu" "F.Mask" "F.Paste") (roundrect_rratio 0.15) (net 2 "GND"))
  (pad "79" smd roundrect (at -1 -1.2) (size 0.45 0.3) (layers "F.Cu" "F.Mask" "F.Paste") (roundrect_rratio 0.15) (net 2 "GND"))
  (pad "80" smd roundrect (at 0 -1.2) (size 0.45 0.3) (layers "F.Cu" "F.Mask" "F.Paste") (roundrect_rratio 0.15) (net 2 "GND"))
  (pad "81" smd roundrect (at 1 -1.2) (size 0.45 0.3) (layers "F.Cu" "F.Mask" "F.Paste") (roundrect_rratio 0.15) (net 2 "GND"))
  (pad "82" smd roundrect (at 2 -1.2) (size 0.45 0.3) (layers "F.Cu" "F.Mask" "F.Paste") (roundrect_rratio 0.15) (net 2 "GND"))
  (pad "83" smd roundrect (at -2 0) (size 0.45 0.3) (layers "F.Cu" "F.Mask" "F.Paste") (roundrect_rratio 0.15) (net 2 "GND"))
  (pad "84" smd roundrect (at -1 0) (size 0.45 0.3) (layers "F.Cu" "F.Mask" "F.Paste") (roundrect_rratio 0.15) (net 2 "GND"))
  (pad "85" smd roundrect (at 0 0) (size 0.45 0.3) (layers "F.Cu" "F.Mask" "F.Paste") (roundrect_rratio 0.15) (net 2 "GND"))
  (pad "86" smd roundrect (at 1 0) (size 0.45 0.3) (layers "F.Cu" "F.Mask" "F.Paste") (roundrect_rratio 0.15) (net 2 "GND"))
  (pad "87" smd roundrect (at 2 0) (size 0.45 0.3) (layers "F.Cu" "F.Mask" "F.Paste") (roundrect_rratio 0.15) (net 2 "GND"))
  (pad "88" smd roundrect (at -2 1.2) (size 0.45 0.3) (layers "F.Cu" "F.Mask" "F.Paste") (roundrect_rratio 0.15) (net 2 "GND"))
  (pad "89" smd roundrect (at -1 1.2) (size 0.45 0.3) (layers "F.Cu" "F.Mask" "F.Paste") (roundrect_rratio 0.15) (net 2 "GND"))
  (pad "90" smd roundrect (at 0 1.2) (size 0.45 0.3) (layers "F.Cu" "F.Mask" "F.Paste") (roundrect_rratio 0.15) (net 2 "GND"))
  (pad "91" smd roundrect (at 1 1.2) (size 0.45 0.3) (layers "F.Cu" "F.Mask" "F.Paste") (roundrect_rratio 0.15) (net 2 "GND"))
  (pad "92" smd roundrect (at 2 1.2) (size 0.45 0.3) (layers "F.Cu" "F.Mask" "F.Paste") (roundrect_rratio 0.15) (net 2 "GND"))
  (pad "93" smd roundrect (at -2 2.4) (size 0.45 0.3) (layers "F.Cu" "F.Mask" "F.Paste") (roundrect_rratio 0.15) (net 2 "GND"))
  (pad "94" smd roundrect (at -1 2.4) (size 0.45 0.3) (layers "F.Cu" "F.Mask" "F.Paste") (roundrect_rratio 0.15) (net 2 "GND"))
  (pad "95" smd roundrect (at 0 2.4) (size 0.45 0.3) (layers "F.Cu" "F.Mask" "F.Paste") (roundrect_rratio 0.15) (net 2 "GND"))
  (pad "96" smd roundrect (at 1 2.4) (size 0.45 0.3) (layers "F.Cu" "F.Mask" "F.Paste") (roundrect_rratio 0.15) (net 2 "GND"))
  (pad "97" smd roundrect (at 2 2.4) (size 0.45 0.3) (layers "F.Cu" "F.Mask" "F.Paste") (roundrect_rratio 0.15) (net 2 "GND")))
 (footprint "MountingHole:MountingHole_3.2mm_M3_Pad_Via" (layer "F.Cu") (at 21 166.9)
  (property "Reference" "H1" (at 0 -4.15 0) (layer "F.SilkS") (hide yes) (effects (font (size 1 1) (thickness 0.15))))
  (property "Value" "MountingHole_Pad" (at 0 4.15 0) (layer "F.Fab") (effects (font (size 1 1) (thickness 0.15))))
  (pad "1" thru_hole circle (at -2.4 0) (size 0.8 0.8) (drill 0.5) (layers "*.Cu" "*.Mask") (remove_unused_layers no) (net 2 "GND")
   (zone_connect 2))
  (pad "1" thru_hole circle (at -1.697056 -1.697056) (size 0.8 0.8) (drill 0.5) (layers "*.Cu" "*.Mask") (remove_unused_layers no)
   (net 2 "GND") (zone_connect 2))
  (pad "1" thru_hole circle (at -1.697056 1.697056) (size 0.8 0.8) (drill 0.5) (layers "*.Cu" "*.Mask") (remove_unused_layers no)
   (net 2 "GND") (zone_connect 2))
  (pad "1" thru_hole circle (at 0 -2.4) (size 0.8 0.8) (drill 0.5) (layers "*.Cu" "*.Mask") (remove_unused_layers no) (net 2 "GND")
   (zone_connect 2))
  (pad "1" thru_hole circle (at 0 0) (size 6.4 6.4) (drill 3.2) (layers "*.Cu" "*.Mask") (remove_unused_layers no) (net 2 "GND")
   (zone_connect 2))
  (pad "1" thru_hole circle (at 0 2.4) (size 0.8 0.8) (drill 0.5) (layers "*.Cu" "*.Mask") (remove_unused_layers no) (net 2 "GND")
   (zone_connect 2))
  (pad "1" thru_hole circle (at 1.697056 -1.697056) (size 0.8 0.8) (drill 0.5) (layers "*.Cu" "*.Mask") (remove_unused_layers no)
   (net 2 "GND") (zone_connect 2))
  (pad "1" thru_hole circle (at 1.697056 1.697056) (size 0.8 0.8) (drill 0.5) (layers "*.Cu" "*.Mask") (remove_unused_layers no)
   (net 2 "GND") (zone_connect 2))
  (pad "1" thru_hole circle (at 2.4 0) (size 0.8 0.8) (drill 0.5) (layers "*.Cu" "*.Mask") (remove_unused_layers no) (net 2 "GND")
   (zone_connect 2)))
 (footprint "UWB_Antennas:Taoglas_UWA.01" (layer "F.Cu") (at 152.94 65.63 90)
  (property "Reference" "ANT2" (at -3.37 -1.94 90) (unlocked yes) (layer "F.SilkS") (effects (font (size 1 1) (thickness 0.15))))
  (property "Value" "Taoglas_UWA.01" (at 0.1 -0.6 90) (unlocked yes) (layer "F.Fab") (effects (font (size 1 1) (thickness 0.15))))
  (pad "1" smd rect (at -3.37 0.36) (size 1.2 0.3) (layers "F.Cu" "F.Mask" "F.Paste") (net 10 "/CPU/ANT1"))
  (pad "1" smd roundrect (at -0.875269 -1.69032) (size 1.6 0.6) (layers "F.Cu" "F.Mask" "F.Paste") (roundrect_rratio 0.15)
   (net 10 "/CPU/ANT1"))
  (pad "1" smd custom (at -0.87 -1.69 270) (size 0.6 0.6) (layers "F.Cu") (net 10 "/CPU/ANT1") (thermal_bridge_angle 90)
   (options (clearance outline) (anchor circle)) (primitives))
  (pad "1" smd roundrect (at -0.37 1.86 270) (size 1.1 0.6) (layers "F.Cu" "F.Mask" "F.Paste") (roundrect_rratio 0.15) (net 10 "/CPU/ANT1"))
  (pad "2" smd roundrect (at 2.3 -1.69 270) (size 0.7 1.6) (layers "F.Cu" "F.Mask" "F.Paste") (roundrect_rratio 0.15) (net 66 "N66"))
  (pad "3" smd roundrect (at -1.745 1.86 270) (size 1.1 0.6) (layers "F.Cu" "F.Mask" "F.Paste") (roundrect_rratio 0.15) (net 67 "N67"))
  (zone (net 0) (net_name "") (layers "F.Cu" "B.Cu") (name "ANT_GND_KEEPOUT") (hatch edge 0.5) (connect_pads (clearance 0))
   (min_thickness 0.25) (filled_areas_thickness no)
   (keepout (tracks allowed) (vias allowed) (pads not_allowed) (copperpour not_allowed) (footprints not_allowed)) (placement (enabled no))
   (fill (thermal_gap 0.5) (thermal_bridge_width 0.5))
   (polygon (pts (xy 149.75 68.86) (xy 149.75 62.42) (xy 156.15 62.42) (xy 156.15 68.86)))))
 (gr_rect (start 132 62) (end 172 114) (stroke (width 0.05) (type default)) (fill no) (layer "Edge.Cuts"))
 (segment (start 141.9 77.4) (end 153 77.4) (width 1.2) (layer "F.Cu") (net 10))
 (segment (start 153.3 77.1) (end 153 77.4) (width 1.2) (layer "F.Cu") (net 10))
 (segment (start 140.7 73.9125) (end 140.7 76.2) (width 1.2) (layer "F.Cu") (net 10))
 (segment (start 153.3 69) (end 153.3 77.1) (width 1.2) (layer "F.Cu") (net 10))
 (segment (start 140.7 76.2) (end 141.9 77.4) (width 1.2) (layer "F.Cu") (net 10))
 (segment (start 164 72.9) (end 164 65.07) (width 1.2) (layer "F.Cu") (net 10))
 (segment (start 159.5 77.4) (end 164 72.9) (width 1.2) (layer "F.Cu") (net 10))
 (segment (start 153 77.4) (end 159.5 77.4) (width 1.2) (layer "F.Cu") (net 10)))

